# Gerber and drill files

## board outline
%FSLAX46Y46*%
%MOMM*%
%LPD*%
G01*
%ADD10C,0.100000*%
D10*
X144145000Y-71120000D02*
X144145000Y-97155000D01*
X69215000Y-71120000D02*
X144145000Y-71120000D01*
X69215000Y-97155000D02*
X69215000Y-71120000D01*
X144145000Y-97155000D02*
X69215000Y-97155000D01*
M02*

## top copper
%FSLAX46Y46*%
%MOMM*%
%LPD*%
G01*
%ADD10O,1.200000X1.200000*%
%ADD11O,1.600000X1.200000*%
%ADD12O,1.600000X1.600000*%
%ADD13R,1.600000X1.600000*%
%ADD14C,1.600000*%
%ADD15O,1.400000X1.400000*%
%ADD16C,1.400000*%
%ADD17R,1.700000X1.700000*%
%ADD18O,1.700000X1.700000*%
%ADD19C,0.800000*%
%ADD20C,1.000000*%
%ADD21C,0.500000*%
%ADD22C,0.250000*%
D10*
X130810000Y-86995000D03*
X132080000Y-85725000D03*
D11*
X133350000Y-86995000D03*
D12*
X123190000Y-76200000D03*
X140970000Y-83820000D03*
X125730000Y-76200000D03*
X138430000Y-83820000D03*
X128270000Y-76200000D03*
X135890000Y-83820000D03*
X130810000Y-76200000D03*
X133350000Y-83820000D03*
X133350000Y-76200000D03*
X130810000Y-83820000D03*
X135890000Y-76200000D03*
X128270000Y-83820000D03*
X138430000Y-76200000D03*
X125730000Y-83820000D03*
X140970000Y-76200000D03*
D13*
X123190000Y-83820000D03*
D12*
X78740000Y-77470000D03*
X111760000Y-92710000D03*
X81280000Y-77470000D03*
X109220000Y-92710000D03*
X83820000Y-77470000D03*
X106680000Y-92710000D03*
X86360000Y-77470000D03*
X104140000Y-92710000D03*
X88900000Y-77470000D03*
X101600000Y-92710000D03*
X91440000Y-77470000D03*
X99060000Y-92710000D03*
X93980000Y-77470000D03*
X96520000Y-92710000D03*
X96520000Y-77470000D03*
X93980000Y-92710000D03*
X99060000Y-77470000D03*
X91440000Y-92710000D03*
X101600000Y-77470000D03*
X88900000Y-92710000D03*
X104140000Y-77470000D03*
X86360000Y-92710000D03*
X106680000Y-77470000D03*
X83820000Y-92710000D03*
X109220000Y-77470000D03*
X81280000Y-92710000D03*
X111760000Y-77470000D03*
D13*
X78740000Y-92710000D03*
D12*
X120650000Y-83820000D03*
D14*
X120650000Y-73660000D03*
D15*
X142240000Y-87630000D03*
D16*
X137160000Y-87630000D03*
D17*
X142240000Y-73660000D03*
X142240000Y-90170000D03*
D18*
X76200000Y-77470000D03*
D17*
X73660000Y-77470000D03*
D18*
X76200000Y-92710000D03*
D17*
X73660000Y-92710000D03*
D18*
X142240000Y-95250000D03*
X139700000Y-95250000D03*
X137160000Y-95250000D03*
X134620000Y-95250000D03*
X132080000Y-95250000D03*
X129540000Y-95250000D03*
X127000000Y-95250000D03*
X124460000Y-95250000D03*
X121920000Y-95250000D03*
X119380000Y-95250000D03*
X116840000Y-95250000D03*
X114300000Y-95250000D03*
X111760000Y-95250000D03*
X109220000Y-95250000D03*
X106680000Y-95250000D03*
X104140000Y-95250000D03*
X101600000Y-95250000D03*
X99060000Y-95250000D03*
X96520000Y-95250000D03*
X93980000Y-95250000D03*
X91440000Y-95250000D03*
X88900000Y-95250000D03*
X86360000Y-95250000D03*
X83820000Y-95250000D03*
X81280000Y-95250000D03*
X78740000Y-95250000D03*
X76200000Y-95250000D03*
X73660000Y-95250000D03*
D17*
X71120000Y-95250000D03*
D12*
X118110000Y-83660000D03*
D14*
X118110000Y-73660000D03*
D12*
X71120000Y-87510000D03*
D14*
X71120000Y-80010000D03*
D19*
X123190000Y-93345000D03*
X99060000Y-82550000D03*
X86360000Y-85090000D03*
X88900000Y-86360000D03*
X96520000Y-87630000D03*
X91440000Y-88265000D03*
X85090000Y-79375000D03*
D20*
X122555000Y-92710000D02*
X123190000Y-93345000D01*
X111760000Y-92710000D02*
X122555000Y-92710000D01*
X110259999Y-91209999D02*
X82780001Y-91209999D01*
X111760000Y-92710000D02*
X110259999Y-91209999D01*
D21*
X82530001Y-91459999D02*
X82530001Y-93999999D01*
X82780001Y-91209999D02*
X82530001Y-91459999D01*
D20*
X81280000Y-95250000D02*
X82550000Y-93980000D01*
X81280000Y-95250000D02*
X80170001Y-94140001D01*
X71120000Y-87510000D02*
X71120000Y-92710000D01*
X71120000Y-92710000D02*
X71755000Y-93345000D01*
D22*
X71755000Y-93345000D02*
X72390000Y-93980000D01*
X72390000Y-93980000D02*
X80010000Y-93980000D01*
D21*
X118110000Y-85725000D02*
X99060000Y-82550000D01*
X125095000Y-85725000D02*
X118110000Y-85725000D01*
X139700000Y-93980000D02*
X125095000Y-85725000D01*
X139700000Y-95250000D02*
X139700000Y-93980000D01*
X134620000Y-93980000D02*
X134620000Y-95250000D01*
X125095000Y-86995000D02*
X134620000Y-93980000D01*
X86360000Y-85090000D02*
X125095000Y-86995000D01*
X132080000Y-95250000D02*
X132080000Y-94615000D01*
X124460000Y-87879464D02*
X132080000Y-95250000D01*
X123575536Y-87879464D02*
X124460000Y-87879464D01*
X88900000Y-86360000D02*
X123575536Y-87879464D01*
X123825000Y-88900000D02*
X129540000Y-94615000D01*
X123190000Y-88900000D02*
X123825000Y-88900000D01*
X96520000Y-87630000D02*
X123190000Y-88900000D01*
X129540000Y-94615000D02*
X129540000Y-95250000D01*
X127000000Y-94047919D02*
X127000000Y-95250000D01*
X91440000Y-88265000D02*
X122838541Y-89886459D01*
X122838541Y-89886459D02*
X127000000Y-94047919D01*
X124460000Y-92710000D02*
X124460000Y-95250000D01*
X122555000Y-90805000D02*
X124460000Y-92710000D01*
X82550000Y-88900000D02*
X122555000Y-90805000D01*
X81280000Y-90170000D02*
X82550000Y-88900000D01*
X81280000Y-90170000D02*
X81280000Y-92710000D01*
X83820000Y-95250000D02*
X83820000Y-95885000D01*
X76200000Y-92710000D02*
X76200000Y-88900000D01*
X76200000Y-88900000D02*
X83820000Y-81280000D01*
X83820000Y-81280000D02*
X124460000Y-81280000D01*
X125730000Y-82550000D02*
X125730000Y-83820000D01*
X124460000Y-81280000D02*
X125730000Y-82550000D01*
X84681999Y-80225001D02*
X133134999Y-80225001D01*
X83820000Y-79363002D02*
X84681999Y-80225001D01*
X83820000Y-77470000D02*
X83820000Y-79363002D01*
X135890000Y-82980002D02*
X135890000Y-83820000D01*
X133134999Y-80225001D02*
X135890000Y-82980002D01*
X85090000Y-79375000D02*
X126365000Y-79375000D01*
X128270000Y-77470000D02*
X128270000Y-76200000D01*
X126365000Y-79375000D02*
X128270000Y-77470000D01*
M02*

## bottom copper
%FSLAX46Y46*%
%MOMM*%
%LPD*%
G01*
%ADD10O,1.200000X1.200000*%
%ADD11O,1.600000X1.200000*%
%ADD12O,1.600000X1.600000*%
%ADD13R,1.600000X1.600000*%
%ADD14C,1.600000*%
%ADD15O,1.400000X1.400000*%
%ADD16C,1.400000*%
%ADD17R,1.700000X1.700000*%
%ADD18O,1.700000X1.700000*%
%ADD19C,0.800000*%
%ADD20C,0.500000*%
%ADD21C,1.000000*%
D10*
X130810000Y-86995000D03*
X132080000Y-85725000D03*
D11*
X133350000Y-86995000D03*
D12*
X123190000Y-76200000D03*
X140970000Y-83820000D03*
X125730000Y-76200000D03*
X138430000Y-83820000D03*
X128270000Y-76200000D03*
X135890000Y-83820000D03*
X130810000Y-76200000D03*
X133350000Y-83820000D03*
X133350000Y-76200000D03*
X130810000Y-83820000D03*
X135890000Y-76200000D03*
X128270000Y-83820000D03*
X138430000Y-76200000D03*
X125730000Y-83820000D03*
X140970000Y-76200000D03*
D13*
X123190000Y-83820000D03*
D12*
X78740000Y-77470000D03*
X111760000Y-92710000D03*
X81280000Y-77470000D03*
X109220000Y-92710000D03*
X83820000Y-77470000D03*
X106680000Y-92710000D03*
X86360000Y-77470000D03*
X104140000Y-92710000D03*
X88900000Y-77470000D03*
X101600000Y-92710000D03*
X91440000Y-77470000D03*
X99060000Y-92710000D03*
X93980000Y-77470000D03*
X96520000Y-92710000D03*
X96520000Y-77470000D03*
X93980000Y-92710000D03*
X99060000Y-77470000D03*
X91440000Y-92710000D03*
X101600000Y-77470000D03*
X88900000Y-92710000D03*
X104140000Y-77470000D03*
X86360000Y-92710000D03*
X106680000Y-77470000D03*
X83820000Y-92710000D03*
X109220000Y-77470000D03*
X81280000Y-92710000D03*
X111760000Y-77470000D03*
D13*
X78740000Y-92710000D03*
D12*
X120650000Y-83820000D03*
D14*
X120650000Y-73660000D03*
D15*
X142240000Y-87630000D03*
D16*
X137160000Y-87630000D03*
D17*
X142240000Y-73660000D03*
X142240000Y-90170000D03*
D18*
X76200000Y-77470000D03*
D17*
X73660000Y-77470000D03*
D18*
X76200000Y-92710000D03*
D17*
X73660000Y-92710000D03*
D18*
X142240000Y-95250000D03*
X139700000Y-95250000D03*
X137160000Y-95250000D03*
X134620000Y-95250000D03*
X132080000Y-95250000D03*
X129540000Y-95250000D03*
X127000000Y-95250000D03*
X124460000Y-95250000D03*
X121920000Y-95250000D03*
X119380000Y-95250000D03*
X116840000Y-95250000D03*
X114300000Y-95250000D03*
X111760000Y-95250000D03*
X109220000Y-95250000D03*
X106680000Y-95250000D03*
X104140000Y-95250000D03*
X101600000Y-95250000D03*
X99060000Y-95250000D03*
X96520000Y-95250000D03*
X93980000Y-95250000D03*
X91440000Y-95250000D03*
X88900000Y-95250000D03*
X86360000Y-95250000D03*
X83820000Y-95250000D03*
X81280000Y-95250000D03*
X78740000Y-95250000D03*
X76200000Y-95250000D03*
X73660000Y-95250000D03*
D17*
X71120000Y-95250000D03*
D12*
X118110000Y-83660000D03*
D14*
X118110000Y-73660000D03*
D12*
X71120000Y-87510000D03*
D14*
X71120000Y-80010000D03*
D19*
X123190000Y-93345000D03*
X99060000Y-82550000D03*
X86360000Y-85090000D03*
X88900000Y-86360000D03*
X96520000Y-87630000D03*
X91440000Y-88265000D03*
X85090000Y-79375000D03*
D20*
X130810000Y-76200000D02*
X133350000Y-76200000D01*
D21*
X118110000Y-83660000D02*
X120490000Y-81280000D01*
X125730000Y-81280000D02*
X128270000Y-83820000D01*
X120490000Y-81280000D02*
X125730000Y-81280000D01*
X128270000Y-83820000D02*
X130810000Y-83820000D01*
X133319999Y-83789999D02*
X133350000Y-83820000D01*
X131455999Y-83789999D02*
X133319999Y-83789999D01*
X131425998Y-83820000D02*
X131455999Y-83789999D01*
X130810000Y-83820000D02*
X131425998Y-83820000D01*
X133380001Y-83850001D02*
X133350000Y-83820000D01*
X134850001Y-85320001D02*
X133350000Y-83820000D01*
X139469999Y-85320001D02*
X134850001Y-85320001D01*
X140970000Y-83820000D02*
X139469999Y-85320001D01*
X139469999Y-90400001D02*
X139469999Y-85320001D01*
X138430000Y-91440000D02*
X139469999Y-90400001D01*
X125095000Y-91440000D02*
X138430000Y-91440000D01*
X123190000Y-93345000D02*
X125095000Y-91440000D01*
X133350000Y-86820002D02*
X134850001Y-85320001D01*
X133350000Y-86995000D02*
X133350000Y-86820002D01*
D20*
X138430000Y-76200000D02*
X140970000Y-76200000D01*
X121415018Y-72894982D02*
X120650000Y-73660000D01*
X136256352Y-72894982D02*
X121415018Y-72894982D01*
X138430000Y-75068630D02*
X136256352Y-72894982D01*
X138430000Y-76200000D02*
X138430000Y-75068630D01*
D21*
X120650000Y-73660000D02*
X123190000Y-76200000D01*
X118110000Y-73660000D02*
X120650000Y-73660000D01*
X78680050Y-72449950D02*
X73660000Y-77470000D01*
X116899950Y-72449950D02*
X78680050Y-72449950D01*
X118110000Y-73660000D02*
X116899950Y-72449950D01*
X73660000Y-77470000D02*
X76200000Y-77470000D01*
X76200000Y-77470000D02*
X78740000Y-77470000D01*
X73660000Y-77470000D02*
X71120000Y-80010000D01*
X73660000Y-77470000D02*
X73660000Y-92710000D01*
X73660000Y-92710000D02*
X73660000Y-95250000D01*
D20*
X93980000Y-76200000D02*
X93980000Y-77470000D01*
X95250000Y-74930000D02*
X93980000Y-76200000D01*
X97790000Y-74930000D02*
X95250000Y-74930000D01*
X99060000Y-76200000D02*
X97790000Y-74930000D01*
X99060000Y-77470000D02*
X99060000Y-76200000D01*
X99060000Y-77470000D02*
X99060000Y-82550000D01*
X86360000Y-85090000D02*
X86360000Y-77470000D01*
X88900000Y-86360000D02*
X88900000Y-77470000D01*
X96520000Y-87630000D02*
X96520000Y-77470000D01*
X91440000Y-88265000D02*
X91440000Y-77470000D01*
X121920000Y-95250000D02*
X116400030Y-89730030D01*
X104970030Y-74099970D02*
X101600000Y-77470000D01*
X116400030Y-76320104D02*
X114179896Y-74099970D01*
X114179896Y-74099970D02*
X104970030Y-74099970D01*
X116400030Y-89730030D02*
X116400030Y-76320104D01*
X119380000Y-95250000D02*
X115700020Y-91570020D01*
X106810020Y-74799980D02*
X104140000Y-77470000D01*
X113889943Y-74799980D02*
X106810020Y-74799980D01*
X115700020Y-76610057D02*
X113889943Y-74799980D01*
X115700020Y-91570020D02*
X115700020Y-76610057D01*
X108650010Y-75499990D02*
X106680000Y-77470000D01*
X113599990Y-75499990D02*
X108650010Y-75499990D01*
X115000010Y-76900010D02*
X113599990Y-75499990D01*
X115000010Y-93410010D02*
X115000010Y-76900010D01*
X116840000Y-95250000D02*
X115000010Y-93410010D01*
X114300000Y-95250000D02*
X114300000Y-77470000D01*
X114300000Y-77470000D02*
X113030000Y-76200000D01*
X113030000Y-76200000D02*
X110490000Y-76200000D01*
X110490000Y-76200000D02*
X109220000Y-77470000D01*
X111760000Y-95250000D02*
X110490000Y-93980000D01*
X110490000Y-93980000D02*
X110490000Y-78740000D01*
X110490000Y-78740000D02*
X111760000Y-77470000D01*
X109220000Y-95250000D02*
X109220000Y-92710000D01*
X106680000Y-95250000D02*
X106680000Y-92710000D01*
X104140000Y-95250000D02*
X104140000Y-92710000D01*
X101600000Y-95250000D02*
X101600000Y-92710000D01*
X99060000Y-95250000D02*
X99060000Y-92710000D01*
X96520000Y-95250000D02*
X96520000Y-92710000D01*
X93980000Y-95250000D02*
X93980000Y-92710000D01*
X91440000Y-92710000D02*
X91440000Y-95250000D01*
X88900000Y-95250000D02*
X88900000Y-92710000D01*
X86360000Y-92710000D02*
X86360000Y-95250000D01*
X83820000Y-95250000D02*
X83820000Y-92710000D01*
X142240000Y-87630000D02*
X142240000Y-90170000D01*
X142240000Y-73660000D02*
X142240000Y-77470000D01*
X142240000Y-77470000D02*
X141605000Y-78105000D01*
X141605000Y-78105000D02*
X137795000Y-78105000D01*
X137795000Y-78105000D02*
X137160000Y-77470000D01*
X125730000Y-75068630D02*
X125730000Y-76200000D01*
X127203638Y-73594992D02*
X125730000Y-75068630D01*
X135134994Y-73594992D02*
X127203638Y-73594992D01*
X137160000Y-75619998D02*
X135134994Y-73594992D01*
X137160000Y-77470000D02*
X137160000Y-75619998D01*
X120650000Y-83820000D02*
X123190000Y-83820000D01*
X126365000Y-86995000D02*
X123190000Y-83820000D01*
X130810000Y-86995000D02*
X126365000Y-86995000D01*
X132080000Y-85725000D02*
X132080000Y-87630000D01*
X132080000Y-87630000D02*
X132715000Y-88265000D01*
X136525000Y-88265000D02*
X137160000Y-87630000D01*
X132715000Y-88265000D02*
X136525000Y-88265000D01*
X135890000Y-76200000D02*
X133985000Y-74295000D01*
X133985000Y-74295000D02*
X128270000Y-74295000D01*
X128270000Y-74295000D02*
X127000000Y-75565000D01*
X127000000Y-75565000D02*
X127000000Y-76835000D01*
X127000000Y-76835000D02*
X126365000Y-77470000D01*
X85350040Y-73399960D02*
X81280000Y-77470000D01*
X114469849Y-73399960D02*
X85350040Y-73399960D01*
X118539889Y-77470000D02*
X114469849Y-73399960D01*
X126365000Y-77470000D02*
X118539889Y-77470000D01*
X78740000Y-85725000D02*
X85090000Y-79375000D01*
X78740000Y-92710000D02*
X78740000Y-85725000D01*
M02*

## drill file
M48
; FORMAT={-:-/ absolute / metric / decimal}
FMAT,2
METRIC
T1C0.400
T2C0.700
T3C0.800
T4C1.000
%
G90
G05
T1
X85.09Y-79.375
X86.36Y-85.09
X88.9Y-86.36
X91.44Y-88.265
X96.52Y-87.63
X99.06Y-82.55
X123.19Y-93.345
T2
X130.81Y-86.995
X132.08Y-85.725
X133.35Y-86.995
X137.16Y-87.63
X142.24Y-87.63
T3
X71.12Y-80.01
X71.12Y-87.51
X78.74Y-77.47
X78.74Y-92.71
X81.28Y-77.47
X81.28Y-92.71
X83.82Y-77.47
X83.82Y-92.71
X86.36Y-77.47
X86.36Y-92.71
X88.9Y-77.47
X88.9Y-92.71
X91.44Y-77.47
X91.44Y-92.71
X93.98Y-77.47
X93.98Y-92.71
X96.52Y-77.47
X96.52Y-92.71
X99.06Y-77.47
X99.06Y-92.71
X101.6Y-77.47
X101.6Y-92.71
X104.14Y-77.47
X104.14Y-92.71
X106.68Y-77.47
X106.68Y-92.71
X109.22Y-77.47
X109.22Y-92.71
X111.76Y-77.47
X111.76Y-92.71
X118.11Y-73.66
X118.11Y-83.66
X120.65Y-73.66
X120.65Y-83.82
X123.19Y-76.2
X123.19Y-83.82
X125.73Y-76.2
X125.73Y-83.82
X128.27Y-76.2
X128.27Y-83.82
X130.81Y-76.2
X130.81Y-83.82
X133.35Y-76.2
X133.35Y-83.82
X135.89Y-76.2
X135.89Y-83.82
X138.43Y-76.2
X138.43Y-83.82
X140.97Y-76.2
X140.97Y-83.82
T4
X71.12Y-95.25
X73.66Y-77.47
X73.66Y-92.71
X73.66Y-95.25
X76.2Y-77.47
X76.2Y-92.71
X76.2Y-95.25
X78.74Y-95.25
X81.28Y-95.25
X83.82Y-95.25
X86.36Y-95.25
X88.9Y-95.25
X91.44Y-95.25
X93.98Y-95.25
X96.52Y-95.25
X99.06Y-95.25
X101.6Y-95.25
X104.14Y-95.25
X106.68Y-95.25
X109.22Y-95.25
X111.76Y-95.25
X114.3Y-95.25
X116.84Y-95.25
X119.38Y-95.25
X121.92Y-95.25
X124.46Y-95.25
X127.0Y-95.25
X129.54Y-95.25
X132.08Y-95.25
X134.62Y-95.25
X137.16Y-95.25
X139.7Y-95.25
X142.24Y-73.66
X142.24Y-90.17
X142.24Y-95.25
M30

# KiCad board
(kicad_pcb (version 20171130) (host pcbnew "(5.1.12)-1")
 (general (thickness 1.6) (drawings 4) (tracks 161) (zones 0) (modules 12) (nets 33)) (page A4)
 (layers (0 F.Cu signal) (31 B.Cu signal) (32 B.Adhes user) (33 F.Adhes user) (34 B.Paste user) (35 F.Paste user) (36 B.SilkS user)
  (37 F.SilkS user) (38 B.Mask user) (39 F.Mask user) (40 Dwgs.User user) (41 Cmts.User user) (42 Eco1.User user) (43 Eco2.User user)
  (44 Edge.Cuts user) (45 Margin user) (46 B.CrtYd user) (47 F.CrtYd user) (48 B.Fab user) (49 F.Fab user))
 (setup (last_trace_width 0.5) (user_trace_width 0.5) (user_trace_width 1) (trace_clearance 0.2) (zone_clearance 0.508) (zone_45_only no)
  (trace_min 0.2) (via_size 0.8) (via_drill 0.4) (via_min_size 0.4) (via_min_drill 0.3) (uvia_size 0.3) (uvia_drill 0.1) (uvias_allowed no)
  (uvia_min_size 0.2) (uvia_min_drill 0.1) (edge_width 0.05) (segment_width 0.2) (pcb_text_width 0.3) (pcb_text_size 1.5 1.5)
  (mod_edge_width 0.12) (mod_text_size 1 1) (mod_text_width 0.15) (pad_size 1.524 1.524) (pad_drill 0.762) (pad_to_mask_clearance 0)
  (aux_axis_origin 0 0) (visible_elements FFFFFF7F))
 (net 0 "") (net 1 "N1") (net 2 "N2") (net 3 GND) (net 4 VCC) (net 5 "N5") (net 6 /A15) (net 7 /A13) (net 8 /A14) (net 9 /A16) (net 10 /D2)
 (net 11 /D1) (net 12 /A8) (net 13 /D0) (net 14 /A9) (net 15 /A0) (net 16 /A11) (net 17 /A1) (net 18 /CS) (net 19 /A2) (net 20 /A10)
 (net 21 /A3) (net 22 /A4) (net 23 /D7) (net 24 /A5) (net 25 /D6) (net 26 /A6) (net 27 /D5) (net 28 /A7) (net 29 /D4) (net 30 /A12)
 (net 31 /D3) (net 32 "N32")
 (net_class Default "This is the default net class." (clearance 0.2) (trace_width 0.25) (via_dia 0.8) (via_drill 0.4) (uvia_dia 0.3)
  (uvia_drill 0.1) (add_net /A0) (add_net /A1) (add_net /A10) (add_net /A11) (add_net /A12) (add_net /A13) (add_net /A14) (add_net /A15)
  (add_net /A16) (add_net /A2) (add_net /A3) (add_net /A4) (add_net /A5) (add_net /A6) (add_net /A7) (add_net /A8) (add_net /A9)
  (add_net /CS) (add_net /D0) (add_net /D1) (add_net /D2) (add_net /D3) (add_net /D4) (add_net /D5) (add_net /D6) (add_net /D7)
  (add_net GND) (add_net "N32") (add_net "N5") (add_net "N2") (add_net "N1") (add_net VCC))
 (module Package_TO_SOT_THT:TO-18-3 (layer F.Cu) (at 133.35 86.995 180)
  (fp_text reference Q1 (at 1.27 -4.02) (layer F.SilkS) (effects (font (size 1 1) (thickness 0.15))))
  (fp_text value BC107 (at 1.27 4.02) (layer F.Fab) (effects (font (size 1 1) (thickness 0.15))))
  (pad 3 thru_hole oval (at 2.54 0 180) (size 1.2 1.2) (drill 0.7) (layers *.Cu *.Mask) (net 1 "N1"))
  (pad 2 thru_hole oval (at 1.27 1.27 180) (size 1.2 1.2) (drill 0.7) (layers *.Cu *.Mask) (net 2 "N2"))
  (pad 1 thru_hole oval (at 0 0 180) (size 1.6 1.2) (drill 0.7) (layers *.Cu *.Mask) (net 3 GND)))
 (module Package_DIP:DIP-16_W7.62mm (layer F.Cu) (at 123.19 83.82 90)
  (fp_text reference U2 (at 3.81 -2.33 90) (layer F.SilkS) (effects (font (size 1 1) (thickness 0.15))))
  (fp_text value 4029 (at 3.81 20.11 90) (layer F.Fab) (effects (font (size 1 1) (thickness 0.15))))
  (pad 16 thru_hole oval (at 7.62 0 90) (size 1.6 1.6) (drill 0.8) (layers *.Cu *.Mask) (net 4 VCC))
  (pad 8 thru_hole oval (at 0 17.78 90) (size 1.6 1.6) (drill 0.8) (layers *.Cu *.Mask) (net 3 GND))
  (pad 15 thru_hole oval (at 7.62 2.54 90) (size 1.6 1.6) (drill 0.8) (layers *.Cu *.Mask) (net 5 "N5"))
  (pad 7 thru_hole oval (at 0 15.24 90) (size 1.6 1.6) (drill 0.8) (layers *.Cu *.Mask))
  (pad 14 thru_hole oval (at 7.62 5.08 90) (size 1.6 1.6) (drill 0.8) (layers *.Cu *.Mask) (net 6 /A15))
  (pad 6 thru_hole oval (at 0 12.7 90) (size 1.6 1.6) (drill 0.8) (layers *.Cu *.Mask) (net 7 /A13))
  (pad 13 thru_hole oval (at 7.62 7.62 90) (size 1.6 1.6) (drill 0.8) (layers *.Cu *.Mask) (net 3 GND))
  (pad 5 thru_hole oval (at 0 10.16 90) (size 1.6 1.6) (drill 0.8) (layers *.Cu *.Mask) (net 3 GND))
  (pad 12 thru_hole oval (at 7.62 10.16 90) (size 1.6 1.6) (drill 0.8) (layers *.Cu *.Mask) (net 3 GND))
  (pad 4 thru_hole oval (at 0 7.62 90) (size 1.6 1.6) (drill 0.8) (layers *.Cu *.Mask) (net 3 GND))
  (pad 11 thru_hole oval (at 7.62 12.7 90) (size 1.6 1.6) (drill 0.8) (layers *.Cu *.Mask) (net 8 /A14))
  (pad 3 thru_hole oval (at 0 5.08 90) (size 1.6 1.6) (drill 0.8) (layers *.Cu *.Mask) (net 3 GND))
  (pad 10 thru_hole oval (at 7.62 15.24 90) (size 1.6 1.6) (drill 0.8) (layers *.Cu *.Mask) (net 4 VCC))
  (pad 2 thru_hole oval (at 0 2.54 90) (size 1.6 1.6) (drill 0.8) (layers *.Cu *.Mask) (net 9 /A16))
  (pad 9 thru_hole oval (at 7.62 17.78 90) (size 1.6 1.6) (drill 0.8) (layers *.Cu *.Mask) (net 4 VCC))
  (pad 1 thru_hole rect (at 0 0 90) (size 1.6 1.6) (drill 0.8) (layers *.Cu *.Mask) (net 1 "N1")))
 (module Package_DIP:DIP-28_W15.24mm (layer F.Cu) (at 78.74 92.71 90)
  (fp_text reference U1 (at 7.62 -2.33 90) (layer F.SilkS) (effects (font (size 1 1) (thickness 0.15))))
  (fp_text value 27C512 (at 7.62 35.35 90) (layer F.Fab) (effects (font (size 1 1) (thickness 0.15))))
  (pad 28 thru_hole oval (at 15.24 0 90) (size 1.6 1.6) (drill 0.8) (layers *.Cu *.Mask) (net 4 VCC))
  (pad 14 thru_hole oval (at 0 33.02 90) (size 1.6 1.6) (drill 0.8) (layers *.Cu *.Mask) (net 3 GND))
  (pad 27 thru_hole oval (at 15.24 2.54 90) (size 1.6 1.6) (drill 0.8) (layers *.Cu *.Mask) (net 8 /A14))
  (pad 13 thru_hole oval (at 0 30.48 90) (size 1.6 1.6) (drill 0.8) (layers *.Cu *.Mask) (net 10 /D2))
  (pad 26 thru_hole oval (at 15.24 5.08 90) (size 1.6 1.6) (drill 0.8) (layers *.Cu *.Mask) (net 7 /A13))
  (pad 12 thru_hole oval (at 0 27.94 90) (size 1.6 1.6) (drill 0.8) (layers *.Cu *.Mask) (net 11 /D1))
  (pad 25 thru_hole oval (at 15.24 7.62 90) (size 1.6 1.6) (drill 0.8) (layers *.Cu *.Mask) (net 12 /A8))
  (pad 11 thru_hole oval (at 0 25.4 90) (size 1.6 1.6) (drill 0.8) (layers *.Cu *.Mask) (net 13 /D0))
  (pad 24 thru_hole oval (at 15.24 10.16 90) (size 1.6 1.6) (drill 0.8) (layers *.Cu *.Mask) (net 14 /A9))
  (pad 10 thru_hole oval (at 0 22.86 90) (size 1.6 1.6) (drill 0.8) (layers *.Cu *.Mask) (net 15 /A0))
  (pad 23 thru_hole oval (at 15.24 12.7 90) (size 1.6 1.6) (drill 0.8) (layers *.Cu *.Mask) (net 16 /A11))
  (pad 9 thru_hole oval (at 0 20.32 90) (size 1.6 1.6) (drill 0.8) (layers *.Cu *.Mask) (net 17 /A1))
  (pad 22 thru_hole oval (at 15.24 15.24 90) (size 1.6 1.6) (drill 0.8) (layers *.Cu *.Mask) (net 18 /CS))
  (pad 8 thru_hole oval (at 0 17.78 90) (size 1.6 1.6) (drill 0.8) (layers *.Cu *.Mask) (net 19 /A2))
  (pad 21 thru_hole oval (at 15.24 17.78 90) (size 1.6 1.6) (drill 0.8) (layers *.Cu *.Mask) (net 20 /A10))
  (pad 7 thru_hole oval (at 0 15.24 90) (size 1.6 1.6) (drill 0.8) (layers *.Cu *.Mask) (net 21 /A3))
  (pad 20 thru_hole oval (at 15.24 20.32 90) (size 1.6 1.6) (drill 0.8) (layers *.Cu *.Mask) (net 18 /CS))
  (pad 6 thru_hole oval (at 0 12.7 90) (size 1.6 1.6) (drill 0.8) (layers *.Cu *.Mask) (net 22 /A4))
  (pad 19 thru_hole oval (at 15.24 22.86 90) (size 1.6 1.6) (drill 0.8) (layers *.Cu *.Mask) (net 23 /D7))
  (pad 5 thru_hole oval (at 0 10.16 90) (size 1.6 1.6) (drill 0.8) (layers *.Cu *.Mask) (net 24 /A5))
  (pad 18 thru_hole oval (at 15.24 25.4 90) (size 1.6 1.6) (drill 0.8) (layers *.Cu *.Mask) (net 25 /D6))
  (pad 4 thru_hole oval (at 0 7.62 90) (size 1.6 1.6) (drill 0.8) (layers *.Cu *.Mask) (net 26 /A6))
  (pad 17 thru_hole oval (at 15.24 27.94 90) (size 1.6 1.6) (drill 0.8) (layers *.Cu *.Mask) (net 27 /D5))
  (pad 3 thru_hole oval (at 0 5.08 90) (size 1.6 1.6) (drill 0.8) (layers *.Cu *.Mask) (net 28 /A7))
  (pad 16 thru_hole oval (at 15.24 30.48 90) (size 1.6 1.6) (drill 0.8) (layers *.Cu *.Mask) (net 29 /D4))
  (pad 2 thru_hole oval (at 0 2.54 90) (size 1.6 1.6) (drill 0.8) (layers *.Cu *.Mask) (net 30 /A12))
  (pad 15 thru_hole oval (at 15.24 33.02 90) (size 1.6 1.6) (drill 0.8) (layers *.Cu *.Mask) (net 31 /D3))
  (pad 1 thru_hole rect (at 0 0 90) (size 1.6 1.6) (drill 0.8) (layers *.Cu *.Mask) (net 6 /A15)))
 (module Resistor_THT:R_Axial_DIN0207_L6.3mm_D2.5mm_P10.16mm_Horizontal (layer F.Cu) (at 120.65 73.66 270)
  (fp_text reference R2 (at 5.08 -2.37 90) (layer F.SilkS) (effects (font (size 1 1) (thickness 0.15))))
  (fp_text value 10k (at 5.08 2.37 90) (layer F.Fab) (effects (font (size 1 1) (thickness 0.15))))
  (pad 2 thru_hole oval (at 10.16 0 270) (size 1.6 1.6) (drill 0.8) (layers *.Cu *.Mask) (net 1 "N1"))
  (pad 1 thru_hole circle (at 0 0 270) (size 1.6 1.6) (drill 0.8) (layers *.Cu *.Mask) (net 4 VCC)))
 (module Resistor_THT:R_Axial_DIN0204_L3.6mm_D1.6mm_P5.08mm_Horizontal (layer F.Cu) (at 137.16 87.63)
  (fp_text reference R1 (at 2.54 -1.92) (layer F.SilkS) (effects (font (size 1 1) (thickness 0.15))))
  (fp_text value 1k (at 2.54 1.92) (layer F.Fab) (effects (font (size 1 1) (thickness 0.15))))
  (pad 2 thru_hole oval (at 5.08 0) (size 1.4 1.4) (drill 0.7) (layers *.Cu *.Mask) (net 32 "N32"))
  (pad 1 thru_hole circle (at 0 0) (size 1.4 1.4) (drill 0.7) (layers *.Cu *.Mask) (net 2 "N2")))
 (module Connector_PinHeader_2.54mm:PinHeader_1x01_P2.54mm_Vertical (layer F.Cu) (at 142.24 73.66)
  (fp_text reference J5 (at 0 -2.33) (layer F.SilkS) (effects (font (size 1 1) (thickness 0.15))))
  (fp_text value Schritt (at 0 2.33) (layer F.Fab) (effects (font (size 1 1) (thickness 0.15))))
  (pad 1 thru_hole rect (at 0 0) (size 1.7 1.7) (drill 1) (layers *.Cu *.Mask) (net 5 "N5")))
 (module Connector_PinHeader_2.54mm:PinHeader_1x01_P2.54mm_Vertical (layer F.Cu) (at 142.24 90.17)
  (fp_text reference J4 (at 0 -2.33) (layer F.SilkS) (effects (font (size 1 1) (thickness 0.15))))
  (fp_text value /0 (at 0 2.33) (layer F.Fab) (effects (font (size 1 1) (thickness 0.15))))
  (pad 1 thru_hole rect (at 0 0) (size 1.7 1.7) (drill 1) (layers *.Cu *.Mask) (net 32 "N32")))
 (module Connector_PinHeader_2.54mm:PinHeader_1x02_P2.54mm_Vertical (layer F.Cu) (at 73.66 77.47 90)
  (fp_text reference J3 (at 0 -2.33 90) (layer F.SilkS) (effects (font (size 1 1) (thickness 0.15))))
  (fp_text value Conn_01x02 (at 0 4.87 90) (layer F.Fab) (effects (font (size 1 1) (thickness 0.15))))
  (pad 2 thru_hole oval (at 0 2.54 90) (size 1.7 1.7) (drill 1) (layers *.Cu *.Mask) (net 4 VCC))
  (pad 1 thru_hole rect (at 0 0 90) (size 1.7 1.7) (drill 1) (layers *.Cu *.Mask) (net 4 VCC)))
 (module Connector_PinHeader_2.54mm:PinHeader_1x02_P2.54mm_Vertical (layer F.Cu) (at 73.66 92.71 90)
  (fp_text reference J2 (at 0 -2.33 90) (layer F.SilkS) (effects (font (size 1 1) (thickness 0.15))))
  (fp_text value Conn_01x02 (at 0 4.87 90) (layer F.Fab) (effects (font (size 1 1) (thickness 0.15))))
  (pad 2 thru_hole oval (at 0 2.54 90) (size 1.7 1.7) (drill 1) (layers *.Cu *.Mask) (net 9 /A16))
  (pad 1 thru_hole rect (at 0 0 90) (size 1.7 1.7) (drill 1) (layers *.Cu *.Mask) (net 4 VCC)))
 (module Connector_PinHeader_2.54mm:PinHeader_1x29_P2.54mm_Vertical (layer F.Cu) (at 71.12 95.25 90)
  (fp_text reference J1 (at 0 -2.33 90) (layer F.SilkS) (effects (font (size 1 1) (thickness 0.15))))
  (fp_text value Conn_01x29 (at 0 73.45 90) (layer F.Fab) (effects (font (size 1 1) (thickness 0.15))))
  (pad 29 thru_hole oval (at 0 71.12 90) (size 1.7 1.7) (drill 1) (layers *.Cu *.Mask))
  (pad 28 thru_hole oval (at 0 68.58 90) (size 1.7 1.7) (drill 1) (layers *.Cu *.Mask) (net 18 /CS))
  (pad 27 thru_hole oval (at 0 66.04 90) (size 1.7 1.7) (drill 1) (layers *.Cu *.Mask))
  (pad 26 thru_hole oval (at 0 63.5 90) (size 1.7 1.7) (drill 1) (layers *.Cu *.Mask) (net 12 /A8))
  (pad 25 thru_hole oval (at 0 60.96 90) (size 1.7 1.7) (drill 1) (layers *.Cu *.Mask) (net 14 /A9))
  (pad 24 thru_hole oval (at 0 58.42 90) (size 1.7 1.7) (drill 1) (layers *.Cu *.Mask) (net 20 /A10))
  (pad 23 thru_hole oval (at 0 55.88 90) (size 1.7 1.7) (drill 1) (layers *.Cu *.Mask) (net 16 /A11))
  (pad 22 thru_hole oval (at 0 53.34 90) (size 1.7 1.7) (drill 1) (layers *.Cu *.Mask) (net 30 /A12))
  (pad 21 thru_hole oval (at 0 50.8 90) (size 1.7 1.7) (drill 1) (layers *.Cu *.Mask) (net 23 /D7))
  (pad 20 thru_hole oval (at 0 48.26 90) (size 1.7 1.7) (drill 1) (layers *.Cu *.Mask) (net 25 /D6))
  (pad 19 thru_hole oval (at 0 45.72 90) (size 1.7 1.7) (drill 1) (layers *.Cu *.Mask) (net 27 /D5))
  (pad 18 thru_hole oval (at 0 43.18 90) (size 1.7 1.7) (drill 1) (layers *.Cu *.Mask) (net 29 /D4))
  (pad 17 thru_hole oval (at 0 40.64 90) (size 1.7 1.7) (drill 1) (layers *.Cu *.Mask) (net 31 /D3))
  (pad 16 thru_hole oval (at 0 38.1 90) (size 1.7 1.7) (drill 1) (layers *.Cu *.Mask) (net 10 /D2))
  (pad 15 thru_hole oval (at 0 35.56 90) (size 1.7 1.7) (drill 1) (layers *.Cu *.Mask) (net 11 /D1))
  (pad 14 thru_hole oval (at 0 33.02 90) (size 1.7 1.7) (drill 1) (layers *.Cu *.Mask) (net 13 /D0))
  (pad 13 thru_hole oval (at 0 30.48 90) (size 1.7 1.7) (drill 1) (layers *.Cu *.Mask) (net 15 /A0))
  (pad 12 thru_hole oval (at 0 27.94 90) (size 1.7 1.7) (drill 1) (layers *.Cu *.Mask) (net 17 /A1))
  (pad 11 thru_hole oval (at 0 25.4 90) (size 1.7 1.7) (drill 1) (layers *.Cu *.Mask) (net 19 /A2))
  (pad 10 thru_hole oval (at 0 22.86 90) (size 1.7 1.7) (drill 1) (layers *.Cu *.Mask) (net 21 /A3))
  (pad 9 thru_hole oval (at 0 20.32 90) (size 1.7 1.7) (drill 1) (layers *.Cu *.Mask) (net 22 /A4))
  (pad 8 thru_hole oval (at 0 17.78 90) (size 1.7 1.7) (drill 1) (layers *.Cu *.Mask) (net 24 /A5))
  (pad 7 thru_hole oval (at 0 15.24 90) (size 1.7 1.7) (drill 1) (layers *.Cu *.Mask) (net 26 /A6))
  (pad 6 thru_hole oval (at 0 12.7 90) (size 1.7 1.7) (drill 1) (layers *.Cu *.Mask) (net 28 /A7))
  (pad 5 thru_hole oval (at 0 10.16 90) (size 1.7 1.7) (drill 1) (layers *.Cu *.Mask) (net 3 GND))
  (pad 4 thru_hole oval (at 0 7.62 90) (size 1.7 1.7) (drill 1) (layers *.Cu *.Mask))
  (pad 3 thru_hole oval (at 0 5.08 90) (size 1.7 1.7) (drill 1) (layers *.Cu *.Mask))
  (pad 2 thru_hole oval (at 0 2.54 90) (size 1.7 1.7) (drill 1) (layers *.Cu *.Mask) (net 4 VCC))
  (pad 1 thru_hole rect (at 0 0 90) (size 1.7 1.7) (drill 1) (layers *.Cu *.Mask)))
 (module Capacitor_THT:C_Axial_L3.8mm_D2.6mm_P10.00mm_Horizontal (layer F.Cu) (at 118.11 73.66 270)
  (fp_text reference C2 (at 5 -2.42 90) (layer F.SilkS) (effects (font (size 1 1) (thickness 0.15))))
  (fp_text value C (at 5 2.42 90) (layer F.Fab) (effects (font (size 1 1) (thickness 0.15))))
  (pad 2 thru_hole oval (at 10 0 270) (size 1.6 1.6) (drill 0.8) (layers *.Cu *.Mask) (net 3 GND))
  (pad 1 thru_hole circle (at 0 0 270) (size 1.6 1.6) (drill 0.8) (layers *.Cu *.Mask) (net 4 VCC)))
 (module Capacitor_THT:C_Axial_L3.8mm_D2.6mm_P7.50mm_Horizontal (layer F.Cu) (at 71.12 80.01 270)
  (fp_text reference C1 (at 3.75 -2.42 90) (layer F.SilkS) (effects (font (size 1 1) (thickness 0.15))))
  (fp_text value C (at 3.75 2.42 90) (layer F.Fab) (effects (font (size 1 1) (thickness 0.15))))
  (pad 2 thru_hole oval (at 7.5 0 270) (size 1.6 1.6) (drill 0.8) (layers *.Cu *.Mask) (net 3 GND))
  (pad 1 thru_hole circle (at 0 0 270) (size 1.6 1.6) (drill 0.8) (layers *.Cu *.Mask) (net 4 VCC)))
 (gr_line (start 144.145 71.12) (end 144.145 97.155) (layer Edge.Cuts) (width 0.1))
 (gr_line (start 69.215 71.12) (end 144.145 71.12) (layer Edge.Cuts) (width 0.1))
 (gr_line (start 69.215 97.155) (end 69.215 71.12) (layer Edge.Cuts) (width 0.1))
 (gr_line (start 144.145 97.155) (end 69.215 97.155) (layer Edge.Cuts) (width 0.1))
 (segment (start 130.81 76.2) (end 133.35 76.2) (width 0.5) (layer B.Cu) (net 3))
 (segment (start 118.11 83.66) (end 120.49 81.28) (width 1) (layer B.Cu) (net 3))
 (segment (start 125.73 81.28) (end 128.27 83.82) (width 1) (layer B.Cu) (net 3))
 (segment (start 120.49 81.28) (end 125.73 81.28) (width 1) (layer B.Cu) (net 3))
 (segment (start 128.27 83.82) (end 130.81 83.82) (width 1) (layer B.Cu) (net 3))
 (segment (start 133.319999 83.789999) (end 133.35 83.82) (width 1) (layer B.Cu) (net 3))
 (segment (start 131.455999 83.789999) (end 133.319999 83.789999) (width 1) (layer B.Cu) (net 3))
 (segment (start 131.425998 83.82) (end 131.455999 83.789999) (width 1) (layer B.Cu) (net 3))
 (segment (start 130.81 83.82) (end 131.425998 83.82) (width 1) (layer B.Cu) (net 3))
 (segment (start 133.380001 83.850001) (end 133.35 83.82) (width 1) (layer B.Cu) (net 3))
 (segment (start 134.850001 85.320001) (end 133.35 83.82) (width 1) (layer B.Cu) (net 3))
 (segment (start 139.469999 85.320001) (end 134.850001 85.320001) (width 1) (layer B.Cu) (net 3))
 (segment (start 140.97 83.82) (end 139.469999 85.320001) (width 1) (layer B.Cu) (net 3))
 (via (at 123.19 93.345) (size 0.8) (drill 0.4) (layers F.Cu B.Cu) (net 3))
 (segment (start 122.555 92.71) (end 123.19 93.345) (width 1) (layer F.Cu) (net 3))
 (segment (start 111.76 92.71) (end 122.555 92.71) (width 1) (layer F.Cu) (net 3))
 (segment (start 139.469999 90.400001) (end 139.469999 85.320001) (width 1) (layer B.Cu) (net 3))
 (segment (start 138.43 91.44) (end 139.469999 90.400001) (width 1) (layer B.Cu) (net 3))
 (segment (start 125.095 91.44) (end 138.43 91.44) (width 1) (layer B.Cu) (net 3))
 (segment (start 123.19 93.345) (end 125.095 91.44) (width 1) (layer B.Cu) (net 3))
 (segment (start 110.259999 91.209999) (end 82.780001 91.209999) (width 1) (layer F.Cu) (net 3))
 (segment (start 111.76 92.71) (end 110.259999 91.209999) (width 1) (layer F.Cu) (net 3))
 (segment (start 82.530001 91.459999) (end 82.530001 93.999999) (width 0.5) (layer F.Cu) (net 3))
 (segment (start 82.780001 91.209999) (end 82.530001 91.459999) (width 0.5) (layer F.Cu) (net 3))
 (segment (start 81.28 95.25) (end 82.55 93.98) (width 1) (layer F.Cu) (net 3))
 (segment (start 81.28 95.25) (end 80.170001 94.140001) (width 1) (layer F.Cu) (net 3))
 (segment (start 71.12 87.51) (end 71.12 92.71) (width 1) (layer F.Cu) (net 3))
 (segment (start 71.12 92.71) (end 71.755 93.345) (width 1) (layer F.Cu) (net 3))
 (segment (start 71.755 93.345) (end 72.39 93.98) (width 0.25) (layer F.Cu) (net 3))
 (segment (start 72.39 93.98) (end 80.01 93.98) (width 0.25) (layer F.Cu) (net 3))
 (segment (start 133.35 86.820002) (end 134.850001 85.320001) (width 1) (layer B.Cu) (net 3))
 (segment (start 133.35 86.995) (end 133.35 86.820002) (width 1) (layer B.Cu) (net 3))
 (segment (start 138.43 76.2) (end 140.97 76.2) (width 0.5) (layer B.Cu) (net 4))
 (segment (start 121.415018 72.894982) (end 120.65 73.66) (width 0.5) (layer B.Cu) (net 4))
 (segment (start 136.256352 72.894982) (end 121.415018 72.894982) (width 0.5) (layer B.Cu) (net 4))
 (segment (start 138.43 75.06863) (end 136.256352 72.894982) (width 0.5) (layer B.Cu) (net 4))
 (segment (start 138.43 76.2) (end 138.43 75.06863) (width 0.5) (layer B.Cu) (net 4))
 (segment (start 120.65 73.66) (end 123.19 76.2) (width 1) (layer B.Cu) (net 4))
 (segment (start 118.11 73.66) (end 120.65 73.66) (width 1) (layer B.Cu) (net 4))
 (segment (start 78.68005 72.44995) (end 73.66 77.47) (width 1) (layer B.Cu) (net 4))
 (segment (start 116.89995 72.44995) (end 78.68005 72.44995) (width 1) (layer B.Cu) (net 4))
 (segment (start 118.11 73.66) (end 116.89995 72.44995) (width 1) (layer B.Cu) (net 4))
 (segment (start 73.66 77.47) (end 76.2 77.47) (width 1) (layer B.Cu) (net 4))
 (segment (start 76.2 77.47) (end 78.74 77.47) (width 1) (layer B.Cu) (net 4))
 (segment (start 73.66 77.47) (end 71.12 80.01) (width 1) (layer B.Cu) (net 4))
 (segment (start 73.66 77.47) (end 73.66 92.71) (width 1) (layer B.Cu) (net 4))
 (segment (start 73.66 92.71) (end 73.66 95.25) (width 1) (layer B.Cu) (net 4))
 (segment (start 93.98 76.2) (end 93.98 77.47) (width 0.5) (layer B.Cu) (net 18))
 (segment (start 95.25 74.93) (end 93.98 76.2) (width 0.5) (layer B.Cu) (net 18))
 (segment (start 97.79 74.93) (end 95.25 74.93) (width 0.5) (layer B.Cu) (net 18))
 (segment (start 99.06 76.2) (end 97.79 74.93) (width 0.5) (layer B.Cu) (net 18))
 (segment (start 99.06 77.47) (end 99.06 76.2) (width 0.5) (layer B.Cu) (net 18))
 (via (at 99.06 82.55) (size 0.8) (drill 0.4) (layers F.Cu B.Cu) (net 18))
 (segment (start 99.06 77.47) (end 99.06 82.55) (width 0.5) (layer B.Cu) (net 18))
 (segment (start 118.11 85.725) (end 99.06 82.55) (width 0.5) (layer F.Cu) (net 18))
 (segment (start 125.095 85.725) (end 118.11 85.725) (width 0.5) (layer F.Cu) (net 18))
 (segment (start 139.7 93.98) (end 125.095 85.725) (width 0.5) (layer F.Cu) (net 18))
 (segment (start 139.7 95.25) (end 139.7 93.98) (width 0.5) (layer F.Cu) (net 18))
 (segment (start 134.62 93.98) (end 134.62 95.25) (width 0.5) (layer F.Cu) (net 12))
 (segment (start 125.095 86.995) (end 134.62 93.98) (width 0.5) (layer F.Cu) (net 12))
 (segment (start 86.36 85.09) (end 125.095 86.995) (width 0.5) (layer F.Cu) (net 12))
 (segment (start 86.36 85.09) (end 86.36 77.47) (width 0.5) (layer B.Cu) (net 12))
 (via (at 86.36 85.09) (size 0.8) (drill 0.4) (layers F.Cu B.Cu) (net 12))
 (segment (start 132.08 95.25) (end 132.08 94.615) (width 0.5) (layer F.Cu) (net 14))
 (segment (start 124.46 87.879464) (end 132.08 95.25) (width 0.5) (layer F.Cu) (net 14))
 (segment (start 123.575536 87.879464) (end 124.46 87.879464) (width 0.5) (layer F.Cu) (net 14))
 (segment (start 88.9 86.36) (end 123.575536 87.879464) (width 0.5) (layer F.Cu) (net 14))
 (segment (start 88.9 86.36) (end 88.9 77.47) (width 0.5) (layer B.Cu) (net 14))
 (via (at 88.9 86.36) (size 0.8) (drill 0.4) (layers F.Cu B.Cu) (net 14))
 (segment (start 123.825 88.9) (end 129.54 94.615) (width 0.5) (layer F.Cu) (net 20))
 (segment (start 123.19 88.9) (end 123.825 88.9) (width 0.5) (layer F.Cu) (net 20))
 (segment (start 96.52 87.63) (end 123.19 88.9) (width 0.5) (layer F.Cu) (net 20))
 (segment (start 96.52 87.63) (end 96.52 77.47) (width 0.5) (layer B.Cu) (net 20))
 (segment (start 129.54 94.615) (end 129.54 95.25) (width 0.5) (layer F.Cu) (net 20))
 (via (at 96.52 87.63) (size 0.8) (drill 0.4) (layers F.Cu B.Cu) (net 20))
 (segment (start 127 94.047919) (end 127 95.25) (width 0.5) (layer F.Cu) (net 16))
 (segment (start 91.44 88.265) (end 122.838541 89.886459) (width 0.5) (layer F.Cu) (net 16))
 (segment (start 91.44 88.265) (end 91.44 77.47) (width 0.5) (layer B.Cu) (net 16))
 (segment (start 122.838541 89.886459) (end 127 94.047919) (width 0.5) (layer F.Cu) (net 16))
 (via (at 91.44 88.265) (size 0.8) (drill 0.4) (layers F.Cu B.Cu) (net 16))
 (segment (start 124.46 92.71) (end 124.46 95.25) (width 0.5) (layer F.Cu) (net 30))
 (segment (start 122.555 90.805) (end 124.46 92.71) (width 0.5) (layer F.Cu) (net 30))
 (segment (start 82.55 88.9) (end 122.555 90.805) (width 0.5) (layer F.Cu) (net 30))
 (segment (start 81.28 90.17) (end 82.55 88.9) (width 0.5) (layer F.Cu) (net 30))
 (segment (start 81.28 90.17) (end 81.28 92.71) (width 0.5) (layer F.Cu) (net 30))
 (segment (start 121.92 95.25) (end 116.40003 89.73003) (width 0.5) (layer B.Cu) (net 23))
 (segment (start 104.97003 74.09997) (end 101.6 77.47) (width 0.5) (layer B.Cu) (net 23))
 (segment (start 116.40003 76.320104) (end 114.179896 74.09997) (width 0.5) (layer B.Cu) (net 23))
 (segment (start 114.179896 74.09997) (end 104.97003 74.09997) (width 0.5) (layer B.Cu) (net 23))
 (segment (start 116.40003 89.73003) (end 116.40003 76.320104) (width 0.5) (layer B.Cu) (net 23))
 (segment (start 119.38 95.25) (end 115.70002 91.57002) (width 0.5) (layer B.Cu) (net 25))
 (segment (start 106.81002 74.79998) (end 104.14 77.47) (width 0.5) (layer B.Cu) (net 25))
 (segment (start 113.889943 74.79998) (end 106.81002 74.79998) (width 0.5) (layer B.Cu) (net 25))
 (segment (start 115.70002 76.610057) (end 113.889943 74.79998) (width 0.5) (layer B.Cu) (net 25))
 (segment (start 115.70002 91.57002) (end 115.70002 76.610057) (width 0.5) (layer B.Cu) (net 25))
 (segment (start 108.65001 75.49999) (end 106.68 77.47) (width 0.5) (layer B.Cu) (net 27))
 (segment (start 113.59999 75.49999) (end 108.65001 75.49999) (width 0.5) (layer B.Cu) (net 27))
 (segment (start 115.00001 76.90001) (end 113.59999 75.49999) (width 0.5) (layer B.Cu) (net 27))
 (segment (start 115.00001 93.41001) (end 115.00001 76.90001) (width 0.5) (layer B.Cu) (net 27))
 (segment (start 116.84 95.25) (end 115.00001 93.41001) (width 0.5) (layer B.Cu) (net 27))
 (segment (start 114.3 95.25) (end 114.3 77.47) (width 0.5) (layer B.Cu) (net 29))
 (segment (start 114.3 77.47) (end 113.03 76.2) (width 0.5) (layer B.Cu) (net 29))
 (segment (start 113.03 76.2) (end 110.49 76.2) (width 0.5) (layer B.Cu) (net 29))
 (segment (start 110.49 76.2) (end 109.22 77.47) (width 0.5) (layer B.Cu) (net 29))
 (segment (start 111.76 95.25) (end 110.49 93.98) (width 0.5) (layer B.Cu) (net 31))
 (segment (start 110.49 93.98) (end 110.49 78.74) (width 0.5) (layer B.Cu) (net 31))
 (segment (start 110.49 78.74) (end 111.76 77.47) (width 0.5) (layer B.Cu) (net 31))
 (segment (start 109.22 95.25) (end 109.22 92.71) (width 0.5) (layer B.Cu) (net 10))
 (segment (start 106.68 95.25) (end 106.68 92.71) (width 0.5) (layer B.Cu) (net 11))
 (segment (start 104.14 95.25) (end 104.14 92.71) (width 0.5) (layer B.Cu) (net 13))
 (segment (start 101.6 95.25) (end 101.6 92.71) (width 0.5) (layer B.Cu) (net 15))
 (segment (start 99.06 95.25) (end 99.06 92.71) (width 0.5) (layer B.Cu) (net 17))
 (segment (start 96.52 95.25) (end 96.52 92.71) (width 0.5) (layer B.Cu) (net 19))
 (segment (start 93.98 95.25) (end 93.98 92.71) (width 0.5) (layer B.Cu) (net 21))
 (segment (start 91.44 92.71) (end 91.44 95.25) (width 0.5) (layer B.Cu) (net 22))
 (segment (start 88.9 95.25) (end 88.9 92.71) (width 0.5) (layer B.Cu) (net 24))
 (segment (start 86.36 92.71) (end 86.36 95.25) (width 0.5) (layer B.Cu) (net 26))
 (segment (start 83.82 95.25) (end 83.82 92.71) (width 0.5) (layer B.Cu) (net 28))
 (segment (start 83.82 95.25) (end 83.82 95.885) (width 0.5) (layer F.Cu) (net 28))
 (segment (start 76.2 92.71) (end 76.2 88.9) (width 0.5) (layer F.Cu) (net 9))
 (segment (start 76.2 88.9) (end 83.82 81.28) (width 0.5) (layer F.Cu) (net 9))
 (segment (start 83.82 81.28) (end 124.46 81.28) (width 0.5) (layer F.Cu) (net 9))
 (segment (start 125.73 82.55) (end 125.73 83.82) (width 0.5) (layer F.Cu) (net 9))
 (segment (start 124.46 81.28) (end 125.73 82.55) (width 0.5) (layer F.Cu) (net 9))
 (segment (start 142.24 87.63) (end 142.24 90.17) (width 0.5) (layer B.Cu) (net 32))
 (segment (start 142.24 73.66) (end 142.24 77.47) (width 0.5) (layer B.Cu) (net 5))
 (segment (start 142.24 77.47) (end 141.605 78.105) (width 0.5) (layer B.Cu) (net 5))
 (segment (start 141.605 78.105) (end 137.795 78.105) (width 0.5) (layer B.Cu) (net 5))
 (segment (start 137.795 78.105) (end 137.16 77.47) (width 0.5) (layer B.Cu) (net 5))
 (segment (start 125.73 75.06863) (end 125.73 76.2) (width 0.5) (layer B.Cu) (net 5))
 (segment (start 127.203638 73.594992) (end 125.73 75.06863) (width 0.5) (layer B.Cu) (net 5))
 (segment (start 135.134994 73.594992) (end 127.203638 73.594992) (width 0.5) (layer B.Cu) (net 5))
 (segment (start 137.16 75.619998) (end 135.134994 73.594992) (width 0.5) (layer B.Cu) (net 5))
 (segment (start 137.16 77.47) (end 137.16 75.619998) (width 0.5) (layer B.Cu) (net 5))
 (segment (start 120.65 83.82) (end 123.19 83.82) (width 0.5) (layer B.Cu) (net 1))
 (segment (start 126.365 86.995) (end 123.19 83.82) (width 0.5) (layer B.Cu) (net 1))
 (segment (start 130.81 86.995) (end 126.365 86.995) (width 0.5) (layer B.Cu) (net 1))
 (segment (start 132.08 85.725) (end 132.08 87.63) (width 0.5) (layer B.Cu) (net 2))
 (segment (start 132.08 87.63) (end 132.715 88.265) (width 0.5) (layer B.Cu) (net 2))
 (segment (start 136.525 88.265) (end 137.16 87.63) (width 0.5) (layer B.Cu) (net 2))
 (segment (start 132.715 88.265) (end 136.525 88.265) (width 0.5) (layer B.Cu) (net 2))
 (segment (start 135.89 76.2) (end 133.985 74.295) (width 0.5) (layer B.Cu) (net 8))
 (segment (start 133.985 74.295) (end 128.27 74.295) (width 0.5) (layer B.Cu) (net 8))
 (segment (start 128.27 74.295) (end 127 75.565) (width 0.5) (layer B.Cu) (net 8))
 (segment (start 127 75.565) (end 127 76.835) (width 0.5) (layer B.Cu) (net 8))
 (segment (start 127 76.835) (end 126.365 77.47) (width 0.5) (layer B.Cu) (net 8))
 (segment (start 85.35004 73.39996) (end 81.28 77.47) (width 0.5) (layer B.Cu) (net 8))
 (segment (start 114.469849 73.39996) (end 85.35004 73.39996) (width 0.5) (layer B.Cu) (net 8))
 (segment (start 118.539889 77.47) (end 114.469849 73.39996) (width 0.5) (layer B.Cu) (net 8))
 (segment (start 126.365 77.47) (end 118.539889 77.47) (width 0.5) (layer B.Cu) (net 8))
 (segment (start 84.681999 80.225001) (end 133.134999 80.225001) (width 0.5) (layer F.Cu) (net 7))
 (segment (start 83.82 79.363002) (end 84.681999 80.225001) (width 0.5) (layer F.Cu) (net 7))
 (segment (start 83.82 77.47) (end 83.82 79.363002) (width 0.5) (layer F.Cu) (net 7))
 (segment (start 135.89 82.980002) (end 135.89 83.82) (width 0.5) (layer F.Cu) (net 7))
 (segment (start 133.134999 80.225001) (end 135.89 82.980002) (width 0.5) (layer F.Cu) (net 7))
 (via (at 85.09 79.375) (size 0.8) (drill 0.4) (layers F.Cu B.Cu) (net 6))
 (segment (start 78.74 85.725) (end 85.09 79.375) (width 0.5) (layer B.Cu) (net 6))
 (segment (start 78.74 92.71) (end 78.74 85.725) (width 0.5) (layer B.Cu) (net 6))
 (segment (start 85.09 79.375) (end 126.365 79.375) (width 0.5) (layer F.Cu) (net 6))
 (segment (start 128.27 77.47) (end 128.27 76.2) (width 0.5) (layer F.Cu) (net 6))
 (segment (start 126.365 79.375) (end 128.27 77.47) (width 0.5) (layer F.Cu) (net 6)))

